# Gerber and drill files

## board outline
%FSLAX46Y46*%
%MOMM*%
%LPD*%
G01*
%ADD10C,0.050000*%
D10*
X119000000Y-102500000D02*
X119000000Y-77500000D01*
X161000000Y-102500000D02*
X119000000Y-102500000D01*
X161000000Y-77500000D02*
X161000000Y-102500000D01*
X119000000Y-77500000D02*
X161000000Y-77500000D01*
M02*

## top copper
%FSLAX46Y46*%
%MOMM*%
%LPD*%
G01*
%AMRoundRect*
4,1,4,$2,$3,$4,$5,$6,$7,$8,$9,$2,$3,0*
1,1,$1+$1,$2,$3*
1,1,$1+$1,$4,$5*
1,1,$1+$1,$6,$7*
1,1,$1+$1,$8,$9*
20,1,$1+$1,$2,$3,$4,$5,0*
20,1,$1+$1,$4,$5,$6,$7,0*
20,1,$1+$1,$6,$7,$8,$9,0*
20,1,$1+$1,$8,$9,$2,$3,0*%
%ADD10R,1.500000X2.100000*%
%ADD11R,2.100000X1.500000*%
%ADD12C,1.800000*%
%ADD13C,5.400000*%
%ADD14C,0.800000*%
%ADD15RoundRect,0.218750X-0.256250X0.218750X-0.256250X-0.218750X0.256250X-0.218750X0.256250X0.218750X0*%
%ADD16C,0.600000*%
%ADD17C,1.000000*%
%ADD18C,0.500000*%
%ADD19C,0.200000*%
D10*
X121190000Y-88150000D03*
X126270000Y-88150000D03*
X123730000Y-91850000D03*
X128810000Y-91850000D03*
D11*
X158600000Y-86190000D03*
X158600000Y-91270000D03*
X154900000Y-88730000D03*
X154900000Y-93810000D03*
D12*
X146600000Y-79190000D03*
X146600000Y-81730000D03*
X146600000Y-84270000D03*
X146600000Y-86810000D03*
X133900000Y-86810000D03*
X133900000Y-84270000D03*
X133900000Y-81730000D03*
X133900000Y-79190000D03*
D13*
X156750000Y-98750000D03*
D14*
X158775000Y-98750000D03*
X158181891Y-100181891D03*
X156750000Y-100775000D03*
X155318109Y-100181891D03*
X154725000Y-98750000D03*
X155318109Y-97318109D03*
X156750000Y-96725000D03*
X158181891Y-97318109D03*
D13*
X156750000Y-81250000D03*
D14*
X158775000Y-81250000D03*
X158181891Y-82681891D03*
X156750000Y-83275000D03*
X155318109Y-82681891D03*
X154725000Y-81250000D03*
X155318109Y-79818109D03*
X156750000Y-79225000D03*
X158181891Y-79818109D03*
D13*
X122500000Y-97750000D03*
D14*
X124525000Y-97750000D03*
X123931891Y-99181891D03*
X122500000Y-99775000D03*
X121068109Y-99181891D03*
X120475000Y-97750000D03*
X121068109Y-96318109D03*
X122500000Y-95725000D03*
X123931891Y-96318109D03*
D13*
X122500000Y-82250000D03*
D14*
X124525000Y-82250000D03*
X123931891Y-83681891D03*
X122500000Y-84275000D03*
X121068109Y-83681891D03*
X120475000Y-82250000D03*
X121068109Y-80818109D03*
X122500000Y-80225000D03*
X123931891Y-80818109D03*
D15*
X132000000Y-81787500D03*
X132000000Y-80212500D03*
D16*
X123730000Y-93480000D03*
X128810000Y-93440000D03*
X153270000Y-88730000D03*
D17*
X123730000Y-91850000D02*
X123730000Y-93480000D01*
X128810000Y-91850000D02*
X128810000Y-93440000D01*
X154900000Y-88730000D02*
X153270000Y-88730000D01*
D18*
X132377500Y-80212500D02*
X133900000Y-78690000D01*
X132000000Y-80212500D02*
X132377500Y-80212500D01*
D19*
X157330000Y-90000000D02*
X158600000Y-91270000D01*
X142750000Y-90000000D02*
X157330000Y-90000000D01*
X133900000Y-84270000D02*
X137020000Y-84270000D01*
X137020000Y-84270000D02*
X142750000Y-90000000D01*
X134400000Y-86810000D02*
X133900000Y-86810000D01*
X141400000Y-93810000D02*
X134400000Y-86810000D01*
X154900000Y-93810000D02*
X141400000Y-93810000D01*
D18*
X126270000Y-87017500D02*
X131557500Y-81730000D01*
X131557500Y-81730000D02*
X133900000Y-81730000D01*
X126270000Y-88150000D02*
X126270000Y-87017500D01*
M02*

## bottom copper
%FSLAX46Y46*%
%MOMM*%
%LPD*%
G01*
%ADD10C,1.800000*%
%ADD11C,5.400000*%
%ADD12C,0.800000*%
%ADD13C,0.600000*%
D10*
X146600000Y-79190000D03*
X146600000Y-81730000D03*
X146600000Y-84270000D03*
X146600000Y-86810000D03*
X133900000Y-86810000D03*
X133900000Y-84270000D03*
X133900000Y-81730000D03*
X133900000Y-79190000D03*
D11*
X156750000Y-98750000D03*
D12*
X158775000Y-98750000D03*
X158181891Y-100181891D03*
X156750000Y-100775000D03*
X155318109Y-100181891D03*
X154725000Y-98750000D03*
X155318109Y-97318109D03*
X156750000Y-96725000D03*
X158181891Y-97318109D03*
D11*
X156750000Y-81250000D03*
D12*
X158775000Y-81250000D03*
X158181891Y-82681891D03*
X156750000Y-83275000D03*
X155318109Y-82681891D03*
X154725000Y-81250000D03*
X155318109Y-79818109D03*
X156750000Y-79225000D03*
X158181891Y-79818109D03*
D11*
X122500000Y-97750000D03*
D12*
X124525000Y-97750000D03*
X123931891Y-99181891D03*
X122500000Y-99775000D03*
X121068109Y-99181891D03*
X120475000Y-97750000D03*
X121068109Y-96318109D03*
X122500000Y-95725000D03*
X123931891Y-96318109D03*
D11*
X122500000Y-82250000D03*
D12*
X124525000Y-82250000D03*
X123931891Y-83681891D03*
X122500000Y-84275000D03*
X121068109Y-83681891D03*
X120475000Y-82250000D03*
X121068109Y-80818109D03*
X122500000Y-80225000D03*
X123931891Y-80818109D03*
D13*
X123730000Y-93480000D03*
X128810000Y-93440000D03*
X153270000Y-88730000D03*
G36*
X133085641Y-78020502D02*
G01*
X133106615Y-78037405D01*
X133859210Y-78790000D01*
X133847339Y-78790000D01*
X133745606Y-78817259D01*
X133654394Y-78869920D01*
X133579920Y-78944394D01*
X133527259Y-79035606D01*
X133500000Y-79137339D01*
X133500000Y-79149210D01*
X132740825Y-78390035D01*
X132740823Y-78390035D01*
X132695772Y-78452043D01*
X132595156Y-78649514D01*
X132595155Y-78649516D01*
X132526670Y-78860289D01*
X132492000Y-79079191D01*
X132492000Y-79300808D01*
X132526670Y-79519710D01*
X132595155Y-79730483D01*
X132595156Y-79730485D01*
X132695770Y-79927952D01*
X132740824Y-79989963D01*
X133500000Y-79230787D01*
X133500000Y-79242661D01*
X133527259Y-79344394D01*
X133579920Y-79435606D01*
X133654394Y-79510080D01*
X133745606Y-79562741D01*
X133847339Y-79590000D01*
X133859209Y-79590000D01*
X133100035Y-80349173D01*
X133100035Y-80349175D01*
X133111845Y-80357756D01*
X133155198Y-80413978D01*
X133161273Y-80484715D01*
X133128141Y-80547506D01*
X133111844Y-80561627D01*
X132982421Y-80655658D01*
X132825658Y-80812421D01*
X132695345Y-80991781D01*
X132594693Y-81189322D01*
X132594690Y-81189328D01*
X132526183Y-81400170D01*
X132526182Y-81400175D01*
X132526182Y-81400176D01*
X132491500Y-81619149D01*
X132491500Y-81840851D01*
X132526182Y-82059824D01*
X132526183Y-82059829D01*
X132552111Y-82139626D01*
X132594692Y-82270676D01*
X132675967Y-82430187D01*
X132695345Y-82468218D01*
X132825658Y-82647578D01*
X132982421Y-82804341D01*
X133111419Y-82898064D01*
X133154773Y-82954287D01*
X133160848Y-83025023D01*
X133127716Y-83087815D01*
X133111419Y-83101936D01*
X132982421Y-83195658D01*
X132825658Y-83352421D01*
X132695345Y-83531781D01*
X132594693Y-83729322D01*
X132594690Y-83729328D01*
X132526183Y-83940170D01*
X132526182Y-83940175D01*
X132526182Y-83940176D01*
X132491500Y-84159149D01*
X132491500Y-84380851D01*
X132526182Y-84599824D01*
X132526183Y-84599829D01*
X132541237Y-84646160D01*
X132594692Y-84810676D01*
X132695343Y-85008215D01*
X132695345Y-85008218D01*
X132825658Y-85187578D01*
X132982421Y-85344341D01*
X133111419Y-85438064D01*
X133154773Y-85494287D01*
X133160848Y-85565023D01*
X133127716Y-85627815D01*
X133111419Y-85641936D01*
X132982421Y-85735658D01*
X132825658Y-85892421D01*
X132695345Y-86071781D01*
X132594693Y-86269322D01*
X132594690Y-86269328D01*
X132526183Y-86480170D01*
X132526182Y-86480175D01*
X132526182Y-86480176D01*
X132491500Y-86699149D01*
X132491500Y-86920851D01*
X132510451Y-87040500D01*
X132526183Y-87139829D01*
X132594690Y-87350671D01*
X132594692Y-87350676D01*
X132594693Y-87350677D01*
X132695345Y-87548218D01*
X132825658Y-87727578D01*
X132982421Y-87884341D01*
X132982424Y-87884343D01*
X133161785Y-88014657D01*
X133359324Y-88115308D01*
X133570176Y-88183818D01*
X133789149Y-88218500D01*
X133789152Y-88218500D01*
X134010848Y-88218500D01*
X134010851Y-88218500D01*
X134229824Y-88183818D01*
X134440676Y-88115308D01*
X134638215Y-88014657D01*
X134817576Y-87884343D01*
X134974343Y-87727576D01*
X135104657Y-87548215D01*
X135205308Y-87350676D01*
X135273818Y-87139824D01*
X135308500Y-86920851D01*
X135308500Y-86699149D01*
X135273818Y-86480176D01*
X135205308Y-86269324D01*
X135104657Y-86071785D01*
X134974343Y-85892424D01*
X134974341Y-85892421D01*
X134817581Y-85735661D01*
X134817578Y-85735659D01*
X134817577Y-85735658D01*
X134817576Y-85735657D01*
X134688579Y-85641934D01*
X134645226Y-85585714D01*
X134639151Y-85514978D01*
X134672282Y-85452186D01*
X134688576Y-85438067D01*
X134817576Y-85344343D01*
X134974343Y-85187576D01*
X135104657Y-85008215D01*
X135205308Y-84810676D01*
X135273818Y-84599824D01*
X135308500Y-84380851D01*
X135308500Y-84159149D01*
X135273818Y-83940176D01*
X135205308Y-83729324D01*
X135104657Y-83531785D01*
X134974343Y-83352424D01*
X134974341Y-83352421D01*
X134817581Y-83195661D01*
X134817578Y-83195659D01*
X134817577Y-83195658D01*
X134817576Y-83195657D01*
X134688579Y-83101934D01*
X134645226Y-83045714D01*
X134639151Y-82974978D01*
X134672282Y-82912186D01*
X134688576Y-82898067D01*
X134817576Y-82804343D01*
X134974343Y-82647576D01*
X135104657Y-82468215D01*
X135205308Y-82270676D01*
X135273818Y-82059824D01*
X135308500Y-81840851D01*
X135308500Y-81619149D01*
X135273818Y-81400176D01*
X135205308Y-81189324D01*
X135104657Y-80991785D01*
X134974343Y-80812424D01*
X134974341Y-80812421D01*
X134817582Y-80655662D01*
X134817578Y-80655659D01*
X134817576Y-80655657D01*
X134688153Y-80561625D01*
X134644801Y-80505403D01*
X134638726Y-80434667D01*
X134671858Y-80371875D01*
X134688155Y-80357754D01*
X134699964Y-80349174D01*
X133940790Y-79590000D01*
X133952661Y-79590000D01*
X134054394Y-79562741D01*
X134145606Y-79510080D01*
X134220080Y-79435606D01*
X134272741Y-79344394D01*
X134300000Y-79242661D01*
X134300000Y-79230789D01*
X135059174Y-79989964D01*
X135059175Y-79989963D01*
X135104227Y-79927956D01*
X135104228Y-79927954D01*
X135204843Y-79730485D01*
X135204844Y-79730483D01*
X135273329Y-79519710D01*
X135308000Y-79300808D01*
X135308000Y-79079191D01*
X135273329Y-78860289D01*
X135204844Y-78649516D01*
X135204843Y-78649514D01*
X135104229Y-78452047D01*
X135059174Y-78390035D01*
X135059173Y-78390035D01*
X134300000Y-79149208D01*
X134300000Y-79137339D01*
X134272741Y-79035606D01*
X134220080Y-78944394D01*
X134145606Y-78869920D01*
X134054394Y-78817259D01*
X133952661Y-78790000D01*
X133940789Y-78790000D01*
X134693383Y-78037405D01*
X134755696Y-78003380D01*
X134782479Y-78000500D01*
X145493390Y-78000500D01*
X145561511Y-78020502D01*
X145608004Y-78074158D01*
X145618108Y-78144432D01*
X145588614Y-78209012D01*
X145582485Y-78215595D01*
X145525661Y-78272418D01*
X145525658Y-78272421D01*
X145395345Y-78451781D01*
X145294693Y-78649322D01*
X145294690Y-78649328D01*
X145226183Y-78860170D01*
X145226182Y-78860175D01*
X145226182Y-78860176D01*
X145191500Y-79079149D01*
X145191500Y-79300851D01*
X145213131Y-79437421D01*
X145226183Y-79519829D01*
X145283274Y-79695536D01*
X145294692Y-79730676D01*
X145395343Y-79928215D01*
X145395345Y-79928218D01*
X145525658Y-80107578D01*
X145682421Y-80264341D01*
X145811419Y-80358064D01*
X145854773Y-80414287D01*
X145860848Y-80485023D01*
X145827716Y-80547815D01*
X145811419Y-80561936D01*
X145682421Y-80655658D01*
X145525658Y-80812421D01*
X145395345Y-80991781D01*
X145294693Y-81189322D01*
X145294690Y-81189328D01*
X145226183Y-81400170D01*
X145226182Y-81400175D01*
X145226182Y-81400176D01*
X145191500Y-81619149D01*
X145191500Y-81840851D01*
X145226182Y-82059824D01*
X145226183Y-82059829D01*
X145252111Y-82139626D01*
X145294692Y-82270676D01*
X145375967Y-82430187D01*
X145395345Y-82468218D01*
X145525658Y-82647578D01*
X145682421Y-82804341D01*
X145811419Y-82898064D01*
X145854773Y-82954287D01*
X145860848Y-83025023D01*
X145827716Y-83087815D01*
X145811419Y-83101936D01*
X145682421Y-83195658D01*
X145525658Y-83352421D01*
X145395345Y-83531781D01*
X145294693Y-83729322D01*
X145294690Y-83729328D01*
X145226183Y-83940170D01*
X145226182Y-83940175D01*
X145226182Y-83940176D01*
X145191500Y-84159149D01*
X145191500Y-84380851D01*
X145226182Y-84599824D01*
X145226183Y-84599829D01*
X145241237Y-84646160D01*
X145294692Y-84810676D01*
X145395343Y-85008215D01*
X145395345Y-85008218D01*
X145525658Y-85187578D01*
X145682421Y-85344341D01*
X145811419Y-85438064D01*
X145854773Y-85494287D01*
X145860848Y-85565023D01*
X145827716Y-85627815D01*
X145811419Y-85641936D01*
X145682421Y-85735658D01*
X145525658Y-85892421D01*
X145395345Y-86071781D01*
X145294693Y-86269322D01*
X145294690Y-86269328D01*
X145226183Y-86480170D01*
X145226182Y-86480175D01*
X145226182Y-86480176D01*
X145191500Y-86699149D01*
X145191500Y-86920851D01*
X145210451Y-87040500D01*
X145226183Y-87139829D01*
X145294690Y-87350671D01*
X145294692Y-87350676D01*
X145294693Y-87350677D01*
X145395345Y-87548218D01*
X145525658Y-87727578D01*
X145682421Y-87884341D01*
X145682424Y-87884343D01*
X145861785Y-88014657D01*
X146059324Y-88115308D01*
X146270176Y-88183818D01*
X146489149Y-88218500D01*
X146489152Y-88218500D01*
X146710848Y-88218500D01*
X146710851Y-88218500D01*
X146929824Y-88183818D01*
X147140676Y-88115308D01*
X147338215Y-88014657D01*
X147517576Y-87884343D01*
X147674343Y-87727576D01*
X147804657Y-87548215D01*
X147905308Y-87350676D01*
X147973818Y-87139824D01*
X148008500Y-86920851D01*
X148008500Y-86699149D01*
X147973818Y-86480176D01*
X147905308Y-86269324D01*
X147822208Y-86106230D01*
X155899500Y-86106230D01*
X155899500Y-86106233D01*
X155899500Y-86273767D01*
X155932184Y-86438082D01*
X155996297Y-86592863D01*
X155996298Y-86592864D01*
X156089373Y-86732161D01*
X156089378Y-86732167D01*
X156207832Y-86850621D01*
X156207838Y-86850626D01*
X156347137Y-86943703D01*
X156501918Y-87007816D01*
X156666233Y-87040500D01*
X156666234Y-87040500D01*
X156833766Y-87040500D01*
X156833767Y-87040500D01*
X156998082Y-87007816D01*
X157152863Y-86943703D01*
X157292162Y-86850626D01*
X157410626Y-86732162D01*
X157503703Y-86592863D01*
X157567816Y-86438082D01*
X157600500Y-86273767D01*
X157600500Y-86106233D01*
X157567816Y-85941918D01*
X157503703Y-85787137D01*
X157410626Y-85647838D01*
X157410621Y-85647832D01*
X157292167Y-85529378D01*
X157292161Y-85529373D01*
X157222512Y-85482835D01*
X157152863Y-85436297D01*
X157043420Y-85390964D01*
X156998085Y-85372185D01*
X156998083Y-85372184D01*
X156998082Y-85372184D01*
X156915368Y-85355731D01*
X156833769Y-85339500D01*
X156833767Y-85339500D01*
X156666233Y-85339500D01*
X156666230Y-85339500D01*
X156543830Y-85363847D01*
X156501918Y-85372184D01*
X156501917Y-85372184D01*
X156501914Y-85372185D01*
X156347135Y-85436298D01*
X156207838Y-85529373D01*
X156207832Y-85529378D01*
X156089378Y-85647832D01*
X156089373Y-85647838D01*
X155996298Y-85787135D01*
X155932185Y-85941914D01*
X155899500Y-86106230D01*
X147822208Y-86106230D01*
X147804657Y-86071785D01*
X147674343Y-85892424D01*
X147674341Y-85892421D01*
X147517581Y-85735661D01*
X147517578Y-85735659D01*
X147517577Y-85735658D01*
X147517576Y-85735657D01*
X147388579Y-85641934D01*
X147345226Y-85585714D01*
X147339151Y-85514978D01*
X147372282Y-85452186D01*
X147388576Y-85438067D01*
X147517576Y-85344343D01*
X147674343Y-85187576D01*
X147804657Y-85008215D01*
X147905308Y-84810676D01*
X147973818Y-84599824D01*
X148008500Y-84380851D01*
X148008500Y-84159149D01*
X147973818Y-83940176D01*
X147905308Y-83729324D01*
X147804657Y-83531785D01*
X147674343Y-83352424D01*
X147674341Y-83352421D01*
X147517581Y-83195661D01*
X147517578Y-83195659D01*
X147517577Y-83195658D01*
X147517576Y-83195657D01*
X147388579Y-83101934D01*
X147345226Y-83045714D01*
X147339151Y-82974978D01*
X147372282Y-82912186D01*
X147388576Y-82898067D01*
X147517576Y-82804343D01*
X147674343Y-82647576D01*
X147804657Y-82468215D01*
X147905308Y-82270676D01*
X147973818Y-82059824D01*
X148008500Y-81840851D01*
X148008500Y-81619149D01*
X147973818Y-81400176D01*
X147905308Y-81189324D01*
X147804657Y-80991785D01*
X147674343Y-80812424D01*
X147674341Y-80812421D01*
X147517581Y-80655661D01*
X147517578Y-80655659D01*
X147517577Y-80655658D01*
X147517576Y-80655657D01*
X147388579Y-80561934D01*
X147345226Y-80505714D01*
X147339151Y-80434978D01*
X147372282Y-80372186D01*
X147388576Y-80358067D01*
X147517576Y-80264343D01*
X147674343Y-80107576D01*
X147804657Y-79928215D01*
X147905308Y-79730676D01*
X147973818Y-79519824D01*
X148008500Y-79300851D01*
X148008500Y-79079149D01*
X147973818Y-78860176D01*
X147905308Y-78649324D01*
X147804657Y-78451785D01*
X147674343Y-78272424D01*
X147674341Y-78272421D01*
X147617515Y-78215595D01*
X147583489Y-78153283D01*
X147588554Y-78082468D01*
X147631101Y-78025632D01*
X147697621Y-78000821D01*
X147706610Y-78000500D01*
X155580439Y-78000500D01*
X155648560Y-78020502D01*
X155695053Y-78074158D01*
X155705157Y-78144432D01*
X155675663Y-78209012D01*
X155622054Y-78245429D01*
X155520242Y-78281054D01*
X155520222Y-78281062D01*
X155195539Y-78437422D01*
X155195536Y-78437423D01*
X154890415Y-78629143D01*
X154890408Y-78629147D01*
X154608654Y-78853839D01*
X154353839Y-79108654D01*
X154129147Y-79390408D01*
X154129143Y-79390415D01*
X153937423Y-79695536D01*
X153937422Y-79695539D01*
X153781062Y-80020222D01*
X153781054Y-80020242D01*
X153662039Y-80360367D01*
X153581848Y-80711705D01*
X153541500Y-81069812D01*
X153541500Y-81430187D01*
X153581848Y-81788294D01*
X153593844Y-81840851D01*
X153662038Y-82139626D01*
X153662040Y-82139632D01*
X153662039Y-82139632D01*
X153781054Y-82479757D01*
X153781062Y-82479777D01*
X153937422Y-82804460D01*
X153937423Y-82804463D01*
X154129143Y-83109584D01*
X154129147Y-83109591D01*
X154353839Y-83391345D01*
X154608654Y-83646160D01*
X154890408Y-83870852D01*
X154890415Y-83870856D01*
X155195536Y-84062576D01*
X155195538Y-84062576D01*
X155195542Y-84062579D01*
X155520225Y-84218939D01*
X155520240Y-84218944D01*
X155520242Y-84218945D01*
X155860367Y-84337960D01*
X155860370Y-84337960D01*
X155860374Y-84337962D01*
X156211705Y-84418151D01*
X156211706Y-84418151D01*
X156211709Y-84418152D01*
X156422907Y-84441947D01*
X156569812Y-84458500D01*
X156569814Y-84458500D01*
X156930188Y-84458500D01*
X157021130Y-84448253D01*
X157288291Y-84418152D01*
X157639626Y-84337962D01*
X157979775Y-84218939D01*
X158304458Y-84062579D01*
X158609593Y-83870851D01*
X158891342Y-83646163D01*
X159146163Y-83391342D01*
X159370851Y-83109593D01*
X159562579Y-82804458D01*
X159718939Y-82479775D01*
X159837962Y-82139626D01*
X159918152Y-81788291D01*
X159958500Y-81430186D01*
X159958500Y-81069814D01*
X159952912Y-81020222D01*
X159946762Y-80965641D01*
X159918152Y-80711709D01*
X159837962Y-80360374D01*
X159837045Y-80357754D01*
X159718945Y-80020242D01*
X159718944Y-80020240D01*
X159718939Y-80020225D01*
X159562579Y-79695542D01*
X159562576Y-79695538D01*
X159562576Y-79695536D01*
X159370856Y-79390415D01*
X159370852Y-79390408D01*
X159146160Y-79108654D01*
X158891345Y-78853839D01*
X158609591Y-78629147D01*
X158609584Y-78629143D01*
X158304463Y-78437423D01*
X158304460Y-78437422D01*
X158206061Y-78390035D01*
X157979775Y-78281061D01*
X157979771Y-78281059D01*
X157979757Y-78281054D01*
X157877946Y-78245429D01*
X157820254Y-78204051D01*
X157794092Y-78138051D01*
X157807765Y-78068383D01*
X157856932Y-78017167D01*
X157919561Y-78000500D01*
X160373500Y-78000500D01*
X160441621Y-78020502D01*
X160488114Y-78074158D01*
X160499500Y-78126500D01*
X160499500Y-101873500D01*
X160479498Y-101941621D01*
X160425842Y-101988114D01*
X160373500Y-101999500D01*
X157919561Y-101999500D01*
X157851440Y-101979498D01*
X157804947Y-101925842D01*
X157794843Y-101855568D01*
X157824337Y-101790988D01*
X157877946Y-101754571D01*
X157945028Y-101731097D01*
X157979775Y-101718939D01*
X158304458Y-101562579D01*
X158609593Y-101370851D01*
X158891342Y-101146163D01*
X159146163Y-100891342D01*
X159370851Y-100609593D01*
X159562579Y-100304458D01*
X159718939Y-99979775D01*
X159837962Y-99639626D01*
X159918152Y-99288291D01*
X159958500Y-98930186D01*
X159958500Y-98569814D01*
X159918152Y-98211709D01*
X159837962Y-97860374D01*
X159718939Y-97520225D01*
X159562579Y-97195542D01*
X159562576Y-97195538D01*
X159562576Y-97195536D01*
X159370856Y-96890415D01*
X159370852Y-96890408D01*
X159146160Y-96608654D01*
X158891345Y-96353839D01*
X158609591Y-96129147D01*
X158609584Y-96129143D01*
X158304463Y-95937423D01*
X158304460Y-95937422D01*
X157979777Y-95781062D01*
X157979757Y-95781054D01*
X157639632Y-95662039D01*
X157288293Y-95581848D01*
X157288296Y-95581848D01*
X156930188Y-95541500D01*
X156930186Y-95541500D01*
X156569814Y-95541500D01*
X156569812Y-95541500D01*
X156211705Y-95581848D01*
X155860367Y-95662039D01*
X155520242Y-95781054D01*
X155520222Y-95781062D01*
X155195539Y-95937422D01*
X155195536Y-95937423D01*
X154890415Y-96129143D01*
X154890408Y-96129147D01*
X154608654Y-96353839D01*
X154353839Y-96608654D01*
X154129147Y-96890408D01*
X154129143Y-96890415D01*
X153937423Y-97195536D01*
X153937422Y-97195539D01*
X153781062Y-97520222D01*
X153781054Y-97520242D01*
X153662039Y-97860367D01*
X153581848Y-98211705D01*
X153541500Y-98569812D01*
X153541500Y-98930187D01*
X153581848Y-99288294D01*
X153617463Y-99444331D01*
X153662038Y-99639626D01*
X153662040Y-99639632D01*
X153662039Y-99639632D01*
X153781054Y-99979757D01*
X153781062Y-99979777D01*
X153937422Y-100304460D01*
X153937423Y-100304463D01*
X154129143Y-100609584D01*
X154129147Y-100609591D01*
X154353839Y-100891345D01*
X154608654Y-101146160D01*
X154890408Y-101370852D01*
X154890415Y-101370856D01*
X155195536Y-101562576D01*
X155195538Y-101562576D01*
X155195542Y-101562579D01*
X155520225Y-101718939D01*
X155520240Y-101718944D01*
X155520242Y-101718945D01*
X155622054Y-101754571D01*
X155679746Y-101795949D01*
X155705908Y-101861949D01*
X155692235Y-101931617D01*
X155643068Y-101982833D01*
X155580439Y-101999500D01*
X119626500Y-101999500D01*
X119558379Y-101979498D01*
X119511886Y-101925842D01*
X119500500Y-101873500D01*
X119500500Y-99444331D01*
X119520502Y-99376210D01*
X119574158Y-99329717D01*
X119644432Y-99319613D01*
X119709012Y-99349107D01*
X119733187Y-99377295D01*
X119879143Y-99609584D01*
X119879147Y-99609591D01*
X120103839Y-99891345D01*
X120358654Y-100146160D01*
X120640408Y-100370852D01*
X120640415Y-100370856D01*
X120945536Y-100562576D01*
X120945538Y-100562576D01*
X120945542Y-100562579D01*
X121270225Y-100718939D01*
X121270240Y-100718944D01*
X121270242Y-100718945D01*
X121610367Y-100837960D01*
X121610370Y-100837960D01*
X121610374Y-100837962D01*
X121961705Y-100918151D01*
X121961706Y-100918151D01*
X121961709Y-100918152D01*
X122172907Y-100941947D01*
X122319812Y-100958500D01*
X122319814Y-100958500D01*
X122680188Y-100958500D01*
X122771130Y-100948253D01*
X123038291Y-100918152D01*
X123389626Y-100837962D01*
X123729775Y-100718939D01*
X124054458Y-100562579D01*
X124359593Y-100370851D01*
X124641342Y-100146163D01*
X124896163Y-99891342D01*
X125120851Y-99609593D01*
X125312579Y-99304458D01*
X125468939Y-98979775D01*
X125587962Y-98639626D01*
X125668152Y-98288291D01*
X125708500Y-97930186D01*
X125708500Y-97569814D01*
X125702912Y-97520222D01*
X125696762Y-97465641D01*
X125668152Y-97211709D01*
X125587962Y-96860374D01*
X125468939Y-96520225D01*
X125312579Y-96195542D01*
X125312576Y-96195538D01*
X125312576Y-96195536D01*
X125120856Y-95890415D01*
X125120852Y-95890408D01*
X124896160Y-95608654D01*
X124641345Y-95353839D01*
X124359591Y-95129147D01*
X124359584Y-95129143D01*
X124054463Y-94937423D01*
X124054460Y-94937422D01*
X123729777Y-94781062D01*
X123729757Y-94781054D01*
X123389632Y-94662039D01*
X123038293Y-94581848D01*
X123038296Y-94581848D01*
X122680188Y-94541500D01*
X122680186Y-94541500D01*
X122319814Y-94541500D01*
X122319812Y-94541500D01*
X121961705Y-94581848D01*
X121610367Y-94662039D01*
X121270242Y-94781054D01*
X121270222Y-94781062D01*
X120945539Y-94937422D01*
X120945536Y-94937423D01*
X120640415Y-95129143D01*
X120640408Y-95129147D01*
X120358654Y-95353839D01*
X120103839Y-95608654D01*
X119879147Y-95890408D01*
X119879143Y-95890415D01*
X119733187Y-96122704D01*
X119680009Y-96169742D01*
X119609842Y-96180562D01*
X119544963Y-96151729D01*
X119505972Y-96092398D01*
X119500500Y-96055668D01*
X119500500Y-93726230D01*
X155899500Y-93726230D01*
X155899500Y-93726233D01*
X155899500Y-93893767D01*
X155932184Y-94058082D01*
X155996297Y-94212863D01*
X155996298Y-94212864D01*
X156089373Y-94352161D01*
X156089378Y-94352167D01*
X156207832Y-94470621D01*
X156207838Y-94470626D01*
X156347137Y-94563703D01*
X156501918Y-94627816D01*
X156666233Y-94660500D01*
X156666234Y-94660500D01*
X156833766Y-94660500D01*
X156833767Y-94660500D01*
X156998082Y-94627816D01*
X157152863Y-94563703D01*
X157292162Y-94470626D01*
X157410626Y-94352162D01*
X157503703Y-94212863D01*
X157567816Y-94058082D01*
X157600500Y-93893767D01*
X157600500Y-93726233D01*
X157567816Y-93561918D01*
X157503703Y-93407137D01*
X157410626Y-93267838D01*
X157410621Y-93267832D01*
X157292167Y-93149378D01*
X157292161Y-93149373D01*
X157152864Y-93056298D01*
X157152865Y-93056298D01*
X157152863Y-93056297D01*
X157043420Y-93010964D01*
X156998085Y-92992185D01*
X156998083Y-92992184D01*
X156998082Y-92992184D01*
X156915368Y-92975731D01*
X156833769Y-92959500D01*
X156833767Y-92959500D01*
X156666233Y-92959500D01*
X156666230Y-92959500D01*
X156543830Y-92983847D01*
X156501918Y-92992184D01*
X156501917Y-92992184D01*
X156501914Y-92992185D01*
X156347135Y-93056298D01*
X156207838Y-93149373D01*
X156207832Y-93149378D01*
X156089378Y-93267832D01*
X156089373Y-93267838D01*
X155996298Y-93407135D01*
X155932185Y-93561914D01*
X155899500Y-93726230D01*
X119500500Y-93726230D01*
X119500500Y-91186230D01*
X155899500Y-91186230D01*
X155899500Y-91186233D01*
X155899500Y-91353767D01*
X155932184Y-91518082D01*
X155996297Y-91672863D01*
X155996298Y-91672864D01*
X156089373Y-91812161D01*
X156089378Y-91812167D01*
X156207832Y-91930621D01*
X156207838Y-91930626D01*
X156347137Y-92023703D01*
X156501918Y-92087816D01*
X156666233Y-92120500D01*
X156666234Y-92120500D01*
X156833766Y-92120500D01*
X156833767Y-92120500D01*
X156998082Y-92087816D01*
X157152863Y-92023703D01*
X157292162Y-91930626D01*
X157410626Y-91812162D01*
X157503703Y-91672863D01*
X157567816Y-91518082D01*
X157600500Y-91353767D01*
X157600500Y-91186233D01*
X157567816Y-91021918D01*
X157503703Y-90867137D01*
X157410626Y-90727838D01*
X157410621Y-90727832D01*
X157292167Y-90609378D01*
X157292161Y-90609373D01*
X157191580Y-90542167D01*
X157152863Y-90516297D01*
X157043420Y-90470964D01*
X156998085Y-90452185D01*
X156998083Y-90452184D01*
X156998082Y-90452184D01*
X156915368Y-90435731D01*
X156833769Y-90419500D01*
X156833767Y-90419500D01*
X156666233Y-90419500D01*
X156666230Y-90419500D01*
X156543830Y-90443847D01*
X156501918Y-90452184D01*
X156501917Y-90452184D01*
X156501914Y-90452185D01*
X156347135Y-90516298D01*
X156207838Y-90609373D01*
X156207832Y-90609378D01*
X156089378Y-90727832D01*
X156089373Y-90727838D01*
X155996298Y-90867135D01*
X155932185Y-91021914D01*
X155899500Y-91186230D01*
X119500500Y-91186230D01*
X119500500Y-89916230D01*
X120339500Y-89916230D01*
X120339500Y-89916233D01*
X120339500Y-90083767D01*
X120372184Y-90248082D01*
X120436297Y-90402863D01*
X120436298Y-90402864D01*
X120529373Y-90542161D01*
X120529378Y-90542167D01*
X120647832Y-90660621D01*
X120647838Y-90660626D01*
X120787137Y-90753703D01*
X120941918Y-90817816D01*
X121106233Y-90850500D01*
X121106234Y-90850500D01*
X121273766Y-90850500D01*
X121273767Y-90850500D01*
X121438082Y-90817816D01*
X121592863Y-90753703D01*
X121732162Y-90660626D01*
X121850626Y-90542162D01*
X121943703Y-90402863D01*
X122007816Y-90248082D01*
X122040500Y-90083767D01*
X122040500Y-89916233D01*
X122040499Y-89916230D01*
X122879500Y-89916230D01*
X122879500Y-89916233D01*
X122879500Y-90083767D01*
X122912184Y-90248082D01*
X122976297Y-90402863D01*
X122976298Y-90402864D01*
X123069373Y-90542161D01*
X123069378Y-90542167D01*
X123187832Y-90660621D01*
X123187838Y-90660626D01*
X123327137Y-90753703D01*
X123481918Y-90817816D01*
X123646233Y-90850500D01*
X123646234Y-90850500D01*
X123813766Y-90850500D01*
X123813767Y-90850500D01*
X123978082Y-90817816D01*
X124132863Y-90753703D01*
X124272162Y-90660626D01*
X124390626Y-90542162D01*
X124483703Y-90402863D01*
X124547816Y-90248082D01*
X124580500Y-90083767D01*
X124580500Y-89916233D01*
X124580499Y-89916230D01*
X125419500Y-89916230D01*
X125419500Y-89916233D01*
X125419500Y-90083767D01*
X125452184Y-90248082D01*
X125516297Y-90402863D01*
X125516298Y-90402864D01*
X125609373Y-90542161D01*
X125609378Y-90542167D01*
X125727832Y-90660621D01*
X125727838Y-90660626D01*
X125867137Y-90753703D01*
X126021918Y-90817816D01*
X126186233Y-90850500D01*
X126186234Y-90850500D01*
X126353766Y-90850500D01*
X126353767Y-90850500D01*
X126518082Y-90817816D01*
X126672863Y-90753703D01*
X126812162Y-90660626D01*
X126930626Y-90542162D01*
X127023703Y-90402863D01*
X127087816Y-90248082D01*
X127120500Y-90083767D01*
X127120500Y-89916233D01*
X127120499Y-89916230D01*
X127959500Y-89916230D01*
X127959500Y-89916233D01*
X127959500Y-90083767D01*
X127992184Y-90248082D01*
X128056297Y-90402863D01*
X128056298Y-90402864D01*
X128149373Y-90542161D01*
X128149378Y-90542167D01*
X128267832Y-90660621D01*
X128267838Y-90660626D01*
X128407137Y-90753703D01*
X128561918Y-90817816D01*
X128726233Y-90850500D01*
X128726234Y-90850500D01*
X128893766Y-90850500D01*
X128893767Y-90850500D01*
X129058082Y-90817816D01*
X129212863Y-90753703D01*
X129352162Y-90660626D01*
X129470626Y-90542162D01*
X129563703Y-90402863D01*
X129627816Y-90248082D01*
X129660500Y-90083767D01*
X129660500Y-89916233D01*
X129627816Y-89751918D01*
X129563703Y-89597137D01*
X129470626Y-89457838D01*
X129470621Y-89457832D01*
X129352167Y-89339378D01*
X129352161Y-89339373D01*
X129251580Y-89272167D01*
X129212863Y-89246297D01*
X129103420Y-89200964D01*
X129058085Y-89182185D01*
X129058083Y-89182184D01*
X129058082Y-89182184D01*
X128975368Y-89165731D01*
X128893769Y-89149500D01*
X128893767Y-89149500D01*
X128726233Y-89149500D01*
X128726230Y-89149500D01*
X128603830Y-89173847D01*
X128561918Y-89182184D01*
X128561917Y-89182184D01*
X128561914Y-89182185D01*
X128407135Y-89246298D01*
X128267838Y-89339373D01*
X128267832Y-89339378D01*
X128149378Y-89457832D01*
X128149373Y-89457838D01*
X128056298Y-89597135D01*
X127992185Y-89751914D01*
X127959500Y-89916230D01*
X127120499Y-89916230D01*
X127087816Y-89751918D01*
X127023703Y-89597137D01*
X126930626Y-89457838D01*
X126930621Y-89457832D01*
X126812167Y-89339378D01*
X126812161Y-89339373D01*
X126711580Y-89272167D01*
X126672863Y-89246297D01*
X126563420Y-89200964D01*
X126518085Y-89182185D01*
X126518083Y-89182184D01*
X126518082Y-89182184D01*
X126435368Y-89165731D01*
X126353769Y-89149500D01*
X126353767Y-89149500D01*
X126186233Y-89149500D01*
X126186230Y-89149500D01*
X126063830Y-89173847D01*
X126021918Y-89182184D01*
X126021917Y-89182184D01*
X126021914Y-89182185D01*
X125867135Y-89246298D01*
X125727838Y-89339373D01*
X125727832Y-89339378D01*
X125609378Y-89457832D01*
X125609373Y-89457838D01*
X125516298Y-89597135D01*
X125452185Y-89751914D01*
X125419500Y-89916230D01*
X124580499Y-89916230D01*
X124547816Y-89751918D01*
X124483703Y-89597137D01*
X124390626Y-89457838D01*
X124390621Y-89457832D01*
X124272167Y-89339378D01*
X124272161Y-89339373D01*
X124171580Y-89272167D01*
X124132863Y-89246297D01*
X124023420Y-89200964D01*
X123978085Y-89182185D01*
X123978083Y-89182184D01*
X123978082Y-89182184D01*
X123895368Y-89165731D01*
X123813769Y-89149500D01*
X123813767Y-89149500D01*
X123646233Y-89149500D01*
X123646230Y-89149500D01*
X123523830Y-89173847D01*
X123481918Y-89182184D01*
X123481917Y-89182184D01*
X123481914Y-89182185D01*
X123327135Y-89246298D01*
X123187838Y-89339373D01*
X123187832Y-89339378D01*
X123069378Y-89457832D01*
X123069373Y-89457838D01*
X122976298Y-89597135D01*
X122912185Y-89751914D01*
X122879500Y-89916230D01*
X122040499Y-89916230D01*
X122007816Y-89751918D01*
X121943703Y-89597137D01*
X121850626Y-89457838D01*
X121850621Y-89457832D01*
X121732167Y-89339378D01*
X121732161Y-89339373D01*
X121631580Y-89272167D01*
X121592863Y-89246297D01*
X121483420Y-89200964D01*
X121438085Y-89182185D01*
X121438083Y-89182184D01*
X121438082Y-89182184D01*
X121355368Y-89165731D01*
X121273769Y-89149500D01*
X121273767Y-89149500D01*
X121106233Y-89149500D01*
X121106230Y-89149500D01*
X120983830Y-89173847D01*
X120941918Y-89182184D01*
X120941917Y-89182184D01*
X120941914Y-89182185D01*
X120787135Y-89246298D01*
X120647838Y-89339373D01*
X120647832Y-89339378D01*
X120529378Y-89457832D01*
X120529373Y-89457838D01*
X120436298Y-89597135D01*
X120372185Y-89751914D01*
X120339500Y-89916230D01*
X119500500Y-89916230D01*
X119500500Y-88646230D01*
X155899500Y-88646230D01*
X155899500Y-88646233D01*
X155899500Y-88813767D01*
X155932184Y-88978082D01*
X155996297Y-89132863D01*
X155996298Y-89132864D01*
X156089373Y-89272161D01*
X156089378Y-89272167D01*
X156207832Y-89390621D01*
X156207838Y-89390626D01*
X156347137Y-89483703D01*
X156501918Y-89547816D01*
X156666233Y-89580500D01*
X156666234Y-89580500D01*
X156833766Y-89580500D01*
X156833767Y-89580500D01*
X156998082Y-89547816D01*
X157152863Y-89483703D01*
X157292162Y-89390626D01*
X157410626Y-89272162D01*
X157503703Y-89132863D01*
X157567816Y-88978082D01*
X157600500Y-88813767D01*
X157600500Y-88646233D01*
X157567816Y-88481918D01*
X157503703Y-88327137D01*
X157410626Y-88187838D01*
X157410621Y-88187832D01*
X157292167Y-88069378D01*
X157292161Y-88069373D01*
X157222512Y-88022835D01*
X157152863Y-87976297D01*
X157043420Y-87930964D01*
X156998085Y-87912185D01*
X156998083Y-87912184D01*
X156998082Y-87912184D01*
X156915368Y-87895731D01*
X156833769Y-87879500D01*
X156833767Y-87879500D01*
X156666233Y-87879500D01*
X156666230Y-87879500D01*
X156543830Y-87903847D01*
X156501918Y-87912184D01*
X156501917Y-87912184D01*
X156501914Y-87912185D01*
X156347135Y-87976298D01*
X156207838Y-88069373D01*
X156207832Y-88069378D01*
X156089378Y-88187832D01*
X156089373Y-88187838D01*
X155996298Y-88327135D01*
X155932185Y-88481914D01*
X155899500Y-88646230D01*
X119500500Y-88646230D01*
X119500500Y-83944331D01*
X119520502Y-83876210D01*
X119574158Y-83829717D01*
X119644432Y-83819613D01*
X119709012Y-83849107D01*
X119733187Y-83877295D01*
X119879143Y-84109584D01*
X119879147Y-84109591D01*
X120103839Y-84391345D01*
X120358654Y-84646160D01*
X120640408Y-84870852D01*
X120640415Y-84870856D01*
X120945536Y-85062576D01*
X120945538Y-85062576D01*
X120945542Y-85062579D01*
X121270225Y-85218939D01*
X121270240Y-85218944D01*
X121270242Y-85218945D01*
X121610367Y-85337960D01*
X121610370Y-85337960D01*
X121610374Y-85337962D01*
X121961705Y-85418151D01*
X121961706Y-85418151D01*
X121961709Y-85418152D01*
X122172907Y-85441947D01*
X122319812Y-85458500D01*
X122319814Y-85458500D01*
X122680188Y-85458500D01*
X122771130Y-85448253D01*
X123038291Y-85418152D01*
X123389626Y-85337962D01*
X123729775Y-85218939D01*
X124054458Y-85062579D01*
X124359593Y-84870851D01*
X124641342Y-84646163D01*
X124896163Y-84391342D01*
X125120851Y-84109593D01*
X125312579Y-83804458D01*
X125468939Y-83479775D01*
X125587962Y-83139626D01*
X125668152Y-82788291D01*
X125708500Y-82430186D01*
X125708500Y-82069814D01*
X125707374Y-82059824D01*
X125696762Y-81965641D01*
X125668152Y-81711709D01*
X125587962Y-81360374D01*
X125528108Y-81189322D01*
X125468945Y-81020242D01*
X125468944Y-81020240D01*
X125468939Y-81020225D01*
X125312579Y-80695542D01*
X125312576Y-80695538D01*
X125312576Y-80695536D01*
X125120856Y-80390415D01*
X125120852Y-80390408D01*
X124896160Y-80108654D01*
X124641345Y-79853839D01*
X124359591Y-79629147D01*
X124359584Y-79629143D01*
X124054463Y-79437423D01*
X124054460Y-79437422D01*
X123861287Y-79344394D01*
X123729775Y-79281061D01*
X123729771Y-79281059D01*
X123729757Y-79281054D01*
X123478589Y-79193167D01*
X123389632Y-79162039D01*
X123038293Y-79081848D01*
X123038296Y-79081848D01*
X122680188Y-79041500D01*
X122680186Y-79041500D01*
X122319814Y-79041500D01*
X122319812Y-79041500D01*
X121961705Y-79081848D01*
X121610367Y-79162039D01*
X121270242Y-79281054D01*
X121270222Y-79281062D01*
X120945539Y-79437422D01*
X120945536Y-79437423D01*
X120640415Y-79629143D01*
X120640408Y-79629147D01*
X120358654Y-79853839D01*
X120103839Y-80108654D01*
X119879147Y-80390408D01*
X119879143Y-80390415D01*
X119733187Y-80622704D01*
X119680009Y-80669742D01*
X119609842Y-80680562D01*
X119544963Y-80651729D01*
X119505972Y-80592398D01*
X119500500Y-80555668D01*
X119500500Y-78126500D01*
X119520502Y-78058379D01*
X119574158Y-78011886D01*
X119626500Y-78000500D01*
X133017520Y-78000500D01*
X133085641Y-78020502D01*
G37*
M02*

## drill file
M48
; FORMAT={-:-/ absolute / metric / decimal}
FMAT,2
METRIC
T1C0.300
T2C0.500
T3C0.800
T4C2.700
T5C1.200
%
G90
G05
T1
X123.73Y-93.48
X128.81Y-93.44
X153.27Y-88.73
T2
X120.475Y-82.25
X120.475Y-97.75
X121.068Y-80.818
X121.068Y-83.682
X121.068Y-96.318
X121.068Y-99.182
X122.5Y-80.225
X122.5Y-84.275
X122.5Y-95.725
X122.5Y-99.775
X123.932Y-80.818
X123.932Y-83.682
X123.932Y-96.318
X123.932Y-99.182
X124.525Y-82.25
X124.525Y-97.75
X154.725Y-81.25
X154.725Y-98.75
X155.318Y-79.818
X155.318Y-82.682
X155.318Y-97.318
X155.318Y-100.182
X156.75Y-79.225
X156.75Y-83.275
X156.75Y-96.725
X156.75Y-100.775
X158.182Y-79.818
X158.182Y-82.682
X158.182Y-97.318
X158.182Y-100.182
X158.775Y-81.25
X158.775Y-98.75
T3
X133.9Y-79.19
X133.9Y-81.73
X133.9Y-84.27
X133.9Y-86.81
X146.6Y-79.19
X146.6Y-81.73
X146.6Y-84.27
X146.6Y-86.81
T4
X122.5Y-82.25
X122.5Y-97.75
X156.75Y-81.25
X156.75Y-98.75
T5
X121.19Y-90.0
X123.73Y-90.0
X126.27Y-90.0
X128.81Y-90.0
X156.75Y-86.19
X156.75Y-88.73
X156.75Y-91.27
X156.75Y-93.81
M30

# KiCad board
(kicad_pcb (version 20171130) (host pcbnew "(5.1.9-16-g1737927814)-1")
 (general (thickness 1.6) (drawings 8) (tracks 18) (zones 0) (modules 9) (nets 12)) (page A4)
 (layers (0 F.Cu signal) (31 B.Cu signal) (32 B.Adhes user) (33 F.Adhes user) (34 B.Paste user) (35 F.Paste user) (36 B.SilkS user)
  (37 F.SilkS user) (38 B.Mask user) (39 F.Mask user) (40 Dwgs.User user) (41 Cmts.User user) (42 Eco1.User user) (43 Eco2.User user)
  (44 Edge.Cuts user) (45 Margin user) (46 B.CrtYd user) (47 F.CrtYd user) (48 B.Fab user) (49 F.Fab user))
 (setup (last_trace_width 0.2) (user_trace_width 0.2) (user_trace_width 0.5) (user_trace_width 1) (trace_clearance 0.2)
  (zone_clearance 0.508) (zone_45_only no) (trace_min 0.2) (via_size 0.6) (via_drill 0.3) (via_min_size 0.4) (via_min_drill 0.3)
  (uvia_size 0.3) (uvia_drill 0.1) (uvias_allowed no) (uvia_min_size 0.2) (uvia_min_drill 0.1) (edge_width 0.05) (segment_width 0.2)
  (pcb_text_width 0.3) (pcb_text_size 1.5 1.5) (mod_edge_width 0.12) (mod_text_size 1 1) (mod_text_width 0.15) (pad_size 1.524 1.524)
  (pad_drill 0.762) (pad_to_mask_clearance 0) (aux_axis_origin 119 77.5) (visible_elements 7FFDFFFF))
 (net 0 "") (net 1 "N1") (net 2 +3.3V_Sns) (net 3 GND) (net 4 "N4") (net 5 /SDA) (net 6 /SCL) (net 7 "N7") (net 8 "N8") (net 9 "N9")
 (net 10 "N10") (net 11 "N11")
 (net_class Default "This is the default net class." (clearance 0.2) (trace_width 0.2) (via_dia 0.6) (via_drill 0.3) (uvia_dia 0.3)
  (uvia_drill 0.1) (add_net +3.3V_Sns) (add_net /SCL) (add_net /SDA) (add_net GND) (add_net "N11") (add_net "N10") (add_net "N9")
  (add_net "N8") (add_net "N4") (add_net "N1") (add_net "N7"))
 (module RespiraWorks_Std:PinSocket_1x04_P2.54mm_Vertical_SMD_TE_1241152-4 (layer F.Cu) (at 125 90 90)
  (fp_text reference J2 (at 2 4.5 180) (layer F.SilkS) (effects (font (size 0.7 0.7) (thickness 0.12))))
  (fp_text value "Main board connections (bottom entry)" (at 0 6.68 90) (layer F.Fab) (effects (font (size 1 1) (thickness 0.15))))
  (pad "" np_thru_hole circle (at 0 1.27 90) (size 1.2 1.2) (drill 1.2) (layers *.Cu *.Mask))
  (pad "" np_thru_hole circle (at 0 -1.27 90) (size 1.2 1.2) (drill 1.2) (layers *.Cu *.Mask))
  (pad "" np_thru_hole circle (at 0 -3.81 90) (size 1.2 1.2) (drill 1.2) (layers *.Cu *.Mask))
  (pad 1 smd rect (at 1.85 -3.81 90) (size 2.1 1.5) (layers F.Cu F.Paste F.Mask) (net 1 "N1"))
  (pad 3 smd rect (at 1.85 1.27 90) (size 2.1 1.5) (layers F.Cu F.Paste F.Mask) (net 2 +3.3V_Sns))
  (pad 2 smd rect (at -1.85 -1.27 90) (size 2.1 1.5) (layers F.Cu F.Paste F.Mask) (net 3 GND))
  (pad 4 smd rect (at -1.85 3.81 90) (size 2.1 1.5) (layers F.Cu F.Paste F.Mask) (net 3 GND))
  (pad "" np_thru_hole circle (at 0 3.81 90) (size 1.2 1.2) (drill 1.2) (layers *.Cu *.Mask)))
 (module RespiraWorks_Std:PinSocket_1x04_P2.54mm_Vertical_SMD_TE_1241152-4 (layer F.Cu) (at 156.75 90)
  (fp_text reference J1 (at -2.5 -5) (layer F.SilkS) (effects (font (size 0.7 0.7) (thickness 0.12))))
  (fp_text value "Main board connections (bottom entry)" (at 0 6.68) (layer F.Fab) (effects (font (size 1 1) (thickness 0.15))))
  (pad "" np_thru_hole circle (at 0 1.27) (size 1.2 1.2) (drill 1.2) (layers *.Cu *.Mask))
  (pad "" np_thru_hole circle (at 0 -1.27) (size 1.2 1.2) (drill 1.2) (layers *.Cu *.Mask))
  (pad "" np_thru_hole circle (at 0 -3.81) (size 1.2 1.2) (drill 1.2) (layers *.Cu *.Mask))
  (pad 1 smd rect (at 1.85 -3.81) (size 2.1 1.5) (layers F.Cu F.Paste F.Mask) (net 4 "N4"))
  (pad 3 smd rect (at 1.85 1.27) (size 2.1 1.5) (layers F.Cu F.Paste F.Mask) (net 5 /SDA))
  (pad 2 smd rect (at -1.85 -1.27) (size 2.1 1.5) (layers F.Cu F.Paste F.Mask) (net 3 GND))
  (pad 4 smd rect (at -1.85 3.81) (size 2.1 1.5) (layers F.Cu F.Paste F.Mask) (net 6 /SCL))
  (pad "" np_thru_hole circle (at 0 3.81) (size 1.2 1.2) (drill 1.2) (layers *.Cu *.Mask)))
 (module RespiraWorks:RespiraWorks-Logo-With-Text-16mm (layer B.Cu) (at 140.75 94 270)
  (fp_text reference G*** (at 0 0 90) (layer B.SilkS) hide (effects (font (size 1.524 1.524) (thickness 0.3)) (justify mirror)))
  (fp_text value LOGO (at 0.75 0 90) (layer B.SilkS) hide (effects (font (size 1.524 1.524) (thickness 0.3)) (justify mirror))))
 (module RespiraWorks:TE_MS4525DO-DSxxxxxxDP (layer F.Cu) (at 140.25 83)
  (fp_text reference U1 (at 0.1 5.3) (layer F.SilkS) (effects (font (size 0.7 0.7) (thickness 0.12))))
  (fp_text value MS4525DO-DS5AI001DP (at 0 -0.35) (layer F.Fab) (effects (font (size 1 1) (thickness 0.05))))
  (pad 8 thru_hole circle (at 6.35 -3.81) (size 1.8 1.8) (drill 0.8) (layers *.Cu *.Mask))
  (pad 7 thru_hole circle (at 6.35 -1.27) (size 1.8 1.8) (drill 0.8) (layers *.Cu *.Mask))
  (pad 6 thru_hole circle (at 6.35 1.27) (size 1.8 1.8) (drill 0.8) (layers *.Cu *.Mask))
  (pad 5 thru_hole circle (at 6.35 3.81) (size 1.8 1.8) (drill 0.8) (layers *.Cu *.Mask) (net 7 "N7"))
  (pad 4 thru_hole circle (at -6.35 3.81) (size 1.8 1.8) (drill 0.8) (layers *.Cu *.Mask) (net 6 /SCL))
  (pad 3 thru_hole circle (at -6.35 1.27) (size 1.8 1.8) (drill 0.8) (layers *.Cu *.Mask) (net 5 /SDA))
  (pad 2 thru_hole circle (at -6.35 -1.27) (size 1.8 1.8) (drill 0.8) (layers *.Cu *.Mask) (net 2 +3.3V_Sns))
  (pad 1 thru_hole circle (at -6.35 -3.81) (size 1.8 1.8) (drill 0.8) (layers *.Cu *.Mask) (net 3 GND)))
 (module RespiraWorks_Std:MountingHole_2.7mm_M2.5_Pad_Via (layer F.Cu) (at 156.75 98.75)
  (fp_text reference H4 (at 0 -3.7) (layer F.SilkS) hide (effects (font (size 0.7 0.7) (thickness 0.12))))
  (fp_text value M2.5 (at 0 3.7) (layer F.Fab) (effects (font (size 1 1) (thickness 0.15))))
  (pad 1 thru_hole circle (at 0 0) (size 5.4 5.4) (drill 2.7) (layers *.Cu *.Mask) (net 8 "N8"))
  (pad 1 thru_hole circle (at 2.025 0) (size 0.8 0.8) (drill 0.5) (layers *.Cu *.Mask) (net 8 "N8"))
  (pad 1 thru_hole circle (at 1.431891 1.431891) (size 0.8 0.8) (drill 0.5) (layers *.Cu *.Mask) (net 8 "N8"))
  (pad 1 thru_hole circle (at 0 2.025) (size 0.8 0.8) (drill 0.5) (layers *.Cu *.Mask) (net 8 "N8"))
  (pad 1 thru_hole circle (at -1.431891 1.431891) (size 0.8 0.8) (drill 0.5) (layers *.Cu *.Mask) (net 8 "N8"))
  (pad 1 thru_hole circle (at -2.025 0) (size 0.8 0.8) (drill 0.5) (layers *.Cu *.Mask) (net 8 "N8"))
  (pad 1 thru_hole circle (at -1.431891 -1.431891) (size 0.8 0.8) (drill 0.5) (layers *.Cu *.Mask) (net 8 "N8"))
  (pad 1 thru_hole circle (at 0 -2.025) (size 0.8 0.8) (drill 0.5) (layers *.Cu *.Mask) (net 8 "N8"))
  (pad 1 thru_hole circle (at 1.431891 -1.431891) (size 0.8 0.8) (drill 0.5) (layers *.Cu *.Mask) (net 8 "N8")))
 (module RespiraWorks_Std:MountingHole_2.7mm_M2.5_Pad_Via (layer F.Cu) (at 156.75 81.25)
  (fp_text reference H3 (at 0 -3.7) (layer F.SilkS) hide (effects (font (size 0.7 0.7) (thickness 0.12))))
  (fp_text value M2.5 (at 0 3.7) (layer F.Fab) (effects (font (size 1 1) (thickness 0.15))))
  (pad 1 thru_hole circle (at 0 0) (size 5.4 5.4) (drill 2.7) (layers *.Cu *.Mask) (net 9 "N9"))
  (pad 1 thru_hole circle (at 2.025 0) (size 0.8 0.8) (drill 0.5) (layers *.Cu *.Mask) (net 9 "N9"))
  (pad 1 thru_hole circle (at 1.431891 1.431891) (size 0.8 0.8) (drill 0.5) (layers *.Cu *.Mask) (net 9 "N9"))
  (pad 1 thru_hole circle (at 0 2.025) (size 0.8 0.8) (drill 0.5) (layers *.Cu *.Mask) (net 9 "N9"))
  (pad 1 thru_hole circle (at -1.431891 1.431891) (size 0.8 0.8) (drill 0.5) (layers *.Cu *.Mask) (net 9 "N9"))
  (pad 1 thru_hole circle (at -2.025 0) (size 0.8 0.8) (drill 0.5) (layers *.Cu *.Mask) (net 9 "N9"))
  (pad 1 thru_hole circle (at -1.431891 -1.431891) (size 0.8 0.8) (drill 0.5) (layers *.Cu *.Mask) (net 9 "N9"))
  (pad 1 thru_hole circle (at 0 -2.025) (size 0.8 0.8) (drill 0.5) (layers *.Cu *.Mask) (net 9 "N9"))
  (pad 1 thru_hole circle (at 1.431891 -1.431891) (size 0.8 0.8) (drill 0.5) (layers *.Cu *.Mask) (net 9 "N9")))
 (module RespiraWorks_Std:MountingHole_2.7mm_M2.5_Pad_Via (layer F.Cu) (at 122.5 97.75)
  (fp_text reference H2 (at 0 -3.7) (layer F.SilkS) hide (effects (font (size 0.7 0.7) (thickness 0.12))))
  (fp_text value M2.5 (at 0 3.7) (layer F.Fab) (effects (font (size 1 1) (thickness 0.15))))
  (pad 1 thru_hole circle (at 0 0) (size 5.4 5.4) (drill 2.7) (layers *.Cu *.Mask) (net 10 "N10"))
  (pad 1 thru_hole circle (at 2.025 0) (size 0.8 0.8) (drill 0.5) (layers *.Cu *.Mask) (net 10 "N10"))
  (pad 1 thru_hole circle (at 1.431891 1.431891) (size 0.8 0.8) (drill 0.5) (layers *.Cu *.Mask) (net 10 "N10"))
  (pad 1 thru_hole circle (at 0 2.025) (size 0.8 0.8) (drill 0.5) (layers *.Cu *.Mask) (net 10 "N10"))
  (pad 1 thru_hole circle (at -1.431891 1.431891) (size 0.8 0.8) (drill 0.5) (layers *.Cu *.Mask) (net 10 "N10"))
  (pad 1 thru_hole circle (at -2.025 0) (size 0.8 0.8) (drill 0.5) (layers *.Cu *.Mask) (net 10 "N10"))
  (pad 1 thru_hole circle (at -1.431891 -1.431891) (size 0.8 0.8) (drill 0.5) (layers *.Cu *.Mask) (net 10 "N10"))
  (pad 1 thru_hole circle (at 0 -2.025) (size 0.8 0.8) (drill 0.5) (layers *.Cu *.Mask) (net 10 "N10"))
  (pad 1 thru_hole circle (at 1.431891 -1.431891) (size 0.8 0.8) (drill 0.5) (layers *.Cu *.Mask) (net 10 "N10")))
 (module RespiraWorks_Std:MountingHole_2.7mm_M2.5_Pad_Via (layer F.Cu) (at 122.5 82.25)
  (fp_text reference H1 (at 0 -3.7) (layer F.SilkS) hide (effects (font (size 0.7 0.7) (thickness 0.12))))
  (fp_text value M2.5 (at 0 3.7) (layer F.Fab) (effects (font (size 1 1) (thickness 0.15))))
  (pad 1 thru_hole circle (at 0 0) (size 5.4 5.4) (drill 2.7) (layers *.Cu *.Mask) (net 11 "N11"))
  (pad 1 thru_hole circle (at 2.025 0) (size 0.8 0.8) (drill 0.5) (layers *.Cu *.Mask) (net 11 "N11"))
  (pad 1 thru_hole circle (at 1.431891 1.431891) (size 0.8 0.8) (drill 0.5) (layers *.Cu *.Mask) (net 11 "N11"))
  (pad 1 thru_hole circle (at 0 2.025) (size 0.8 0.8) (drill 0.5) (layers *.Cu *.Mask) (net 11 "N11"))
  (pad 1 thru_hole circle (at -1.431891 1.431891) (size 0.8 0.8) (drill 0.5) (layers *.Cu *.Mask) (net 11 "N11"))
  (pad 1 thru_hole circle (at -2.025 0) (size 0.8 0.8) (drill 0.5) (layers *.Cu *.Mask) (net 11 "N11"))
  (pad 1 thru_hole circle (at -1.431891 -1.431891) (size 0.8 0.8) (drill 0.5) (layers *.Cu *.Mask) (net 11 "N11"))
  (pad 1 thru_hole circle (at 0 -2.025) (size 0.8 0.8) (drill 0.5) (layers *.Cu *.Mask) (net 11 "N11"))
  (pad 1 thru_hole circle (at 1.431891 -1.431891) (size 0.8 0.8) (drill 0.5) (layers *.Cu *.Mask) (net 11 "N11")))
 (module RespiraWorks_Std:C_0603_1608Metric (layer F.Cu) (at 132 81 270)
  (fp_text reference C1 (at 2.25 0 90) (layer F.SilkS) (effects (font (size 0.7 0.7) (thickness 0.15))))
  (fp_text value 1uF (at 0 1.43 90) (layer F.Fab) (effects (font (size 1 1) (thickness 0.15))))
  (pad 2 smd roundrect (at 0.7875 0 270) (size 0.875 0.95) (layers F.Cu F.Paste F.Mask) (roundrect_rratio 0.25) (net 2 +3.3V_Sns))
  (pad 1 smd roundrect (at -0.7875 0 270) (size 0.875 0.95) (layers F.Cu F.Paste F.Mask) (roundrect_rratio 0.25) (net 3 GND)))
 (gr_line (start 119 102.5) (end 119 77.5) (layer Edge.Cuts) (width 0.05))
 (gr_line (start 161 102.5) (end 119 102.5) (layer Edge.Cuts) (width 0.05))
 (gr_line (start 161 77.5) (end 161 102.5) (layer Edge.Cuts) (width 0.05))
 (gr_line (start 119 77.5) (end 161 77.5) (layer Edge.Cuts) (width 0.05))
 (segment (start 123.73 91.85) (end 123.73 93.48) (width 1) (layer F.Cu) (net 3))
 (via (at 123.73 93.48) (size 0.6) (drill 0.3) (layers F.Cu B.Cu) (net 3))
 (segment (start 128.81 91.85) (end 128.81 93.44) (width 1) (layer F.Cu) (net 3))
 (via (at 128.81 93.44) (size 0.6) (drill 0.3) (layers F.Cu B.Cu) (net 3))
 (segment (start 154.9 88.73) (end 153.27 88.73) (width 1) (layer F.Cu) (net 3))
 (via (at 153.27 88.73) (size 0.6) (drill 0.3) (layers F.Cu B.Cu) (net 3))
 (segment (start 132.3775 80.2125) (end 133.9 78.69) (width 0.5) (layer F.Cu) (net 3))
 (segment (start 132 80.2125) (end 132.3775 80.2125) (width 0.5) (layer F.Cu) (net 3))
 (segment (start 157.33 90) (end 158.6 91.27) (width 0.2) (layer F.Cu) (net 5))
 (segment (start 142.75 90) (end 157.33 90) (width 0.2) (layer F.Cu) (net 5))
 (segment (start 133.9 84.27) (end 137.02 84.27) (width 0.2) (layer F.Cu) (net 5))
 (segment (start 137.02 84.27) (end 142.75 90) (width 0.2) (layer F.Cu) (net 5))
 (segment (start 134.4 86.81) (end 133.9 86.81) (width 0.2) (layer F.Cu) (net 6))
 (segment (start 141.4 93.81) (end 134.4 86.81) (width 0.2) (layer F.Cu) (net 6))
 (segment (start 154.9 93.81) (end 141.4 93.81) (width 0.2) (layer F.Cu) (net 6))
 (segment (start 126.27 87.0175) (end 131.5575 81.73) (width 0.5) (layer F.Cu) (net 2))
 (segment (start 131.5575 81.73) (end 133.9 81.73) (width 0.5) (layer F.Cu) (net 2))
 (segment (start 126.27 88.15) (end 126.27 87.0175) (width 0.5) (layer F.Cu) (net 2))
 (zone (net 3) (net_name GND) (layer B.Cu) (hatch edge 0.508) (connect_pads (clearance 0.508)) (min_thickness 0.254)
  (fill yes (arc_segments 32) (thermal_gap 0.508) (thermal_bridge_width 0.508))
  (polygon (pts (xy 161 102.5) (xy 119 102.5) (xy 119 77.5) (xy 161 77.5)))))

